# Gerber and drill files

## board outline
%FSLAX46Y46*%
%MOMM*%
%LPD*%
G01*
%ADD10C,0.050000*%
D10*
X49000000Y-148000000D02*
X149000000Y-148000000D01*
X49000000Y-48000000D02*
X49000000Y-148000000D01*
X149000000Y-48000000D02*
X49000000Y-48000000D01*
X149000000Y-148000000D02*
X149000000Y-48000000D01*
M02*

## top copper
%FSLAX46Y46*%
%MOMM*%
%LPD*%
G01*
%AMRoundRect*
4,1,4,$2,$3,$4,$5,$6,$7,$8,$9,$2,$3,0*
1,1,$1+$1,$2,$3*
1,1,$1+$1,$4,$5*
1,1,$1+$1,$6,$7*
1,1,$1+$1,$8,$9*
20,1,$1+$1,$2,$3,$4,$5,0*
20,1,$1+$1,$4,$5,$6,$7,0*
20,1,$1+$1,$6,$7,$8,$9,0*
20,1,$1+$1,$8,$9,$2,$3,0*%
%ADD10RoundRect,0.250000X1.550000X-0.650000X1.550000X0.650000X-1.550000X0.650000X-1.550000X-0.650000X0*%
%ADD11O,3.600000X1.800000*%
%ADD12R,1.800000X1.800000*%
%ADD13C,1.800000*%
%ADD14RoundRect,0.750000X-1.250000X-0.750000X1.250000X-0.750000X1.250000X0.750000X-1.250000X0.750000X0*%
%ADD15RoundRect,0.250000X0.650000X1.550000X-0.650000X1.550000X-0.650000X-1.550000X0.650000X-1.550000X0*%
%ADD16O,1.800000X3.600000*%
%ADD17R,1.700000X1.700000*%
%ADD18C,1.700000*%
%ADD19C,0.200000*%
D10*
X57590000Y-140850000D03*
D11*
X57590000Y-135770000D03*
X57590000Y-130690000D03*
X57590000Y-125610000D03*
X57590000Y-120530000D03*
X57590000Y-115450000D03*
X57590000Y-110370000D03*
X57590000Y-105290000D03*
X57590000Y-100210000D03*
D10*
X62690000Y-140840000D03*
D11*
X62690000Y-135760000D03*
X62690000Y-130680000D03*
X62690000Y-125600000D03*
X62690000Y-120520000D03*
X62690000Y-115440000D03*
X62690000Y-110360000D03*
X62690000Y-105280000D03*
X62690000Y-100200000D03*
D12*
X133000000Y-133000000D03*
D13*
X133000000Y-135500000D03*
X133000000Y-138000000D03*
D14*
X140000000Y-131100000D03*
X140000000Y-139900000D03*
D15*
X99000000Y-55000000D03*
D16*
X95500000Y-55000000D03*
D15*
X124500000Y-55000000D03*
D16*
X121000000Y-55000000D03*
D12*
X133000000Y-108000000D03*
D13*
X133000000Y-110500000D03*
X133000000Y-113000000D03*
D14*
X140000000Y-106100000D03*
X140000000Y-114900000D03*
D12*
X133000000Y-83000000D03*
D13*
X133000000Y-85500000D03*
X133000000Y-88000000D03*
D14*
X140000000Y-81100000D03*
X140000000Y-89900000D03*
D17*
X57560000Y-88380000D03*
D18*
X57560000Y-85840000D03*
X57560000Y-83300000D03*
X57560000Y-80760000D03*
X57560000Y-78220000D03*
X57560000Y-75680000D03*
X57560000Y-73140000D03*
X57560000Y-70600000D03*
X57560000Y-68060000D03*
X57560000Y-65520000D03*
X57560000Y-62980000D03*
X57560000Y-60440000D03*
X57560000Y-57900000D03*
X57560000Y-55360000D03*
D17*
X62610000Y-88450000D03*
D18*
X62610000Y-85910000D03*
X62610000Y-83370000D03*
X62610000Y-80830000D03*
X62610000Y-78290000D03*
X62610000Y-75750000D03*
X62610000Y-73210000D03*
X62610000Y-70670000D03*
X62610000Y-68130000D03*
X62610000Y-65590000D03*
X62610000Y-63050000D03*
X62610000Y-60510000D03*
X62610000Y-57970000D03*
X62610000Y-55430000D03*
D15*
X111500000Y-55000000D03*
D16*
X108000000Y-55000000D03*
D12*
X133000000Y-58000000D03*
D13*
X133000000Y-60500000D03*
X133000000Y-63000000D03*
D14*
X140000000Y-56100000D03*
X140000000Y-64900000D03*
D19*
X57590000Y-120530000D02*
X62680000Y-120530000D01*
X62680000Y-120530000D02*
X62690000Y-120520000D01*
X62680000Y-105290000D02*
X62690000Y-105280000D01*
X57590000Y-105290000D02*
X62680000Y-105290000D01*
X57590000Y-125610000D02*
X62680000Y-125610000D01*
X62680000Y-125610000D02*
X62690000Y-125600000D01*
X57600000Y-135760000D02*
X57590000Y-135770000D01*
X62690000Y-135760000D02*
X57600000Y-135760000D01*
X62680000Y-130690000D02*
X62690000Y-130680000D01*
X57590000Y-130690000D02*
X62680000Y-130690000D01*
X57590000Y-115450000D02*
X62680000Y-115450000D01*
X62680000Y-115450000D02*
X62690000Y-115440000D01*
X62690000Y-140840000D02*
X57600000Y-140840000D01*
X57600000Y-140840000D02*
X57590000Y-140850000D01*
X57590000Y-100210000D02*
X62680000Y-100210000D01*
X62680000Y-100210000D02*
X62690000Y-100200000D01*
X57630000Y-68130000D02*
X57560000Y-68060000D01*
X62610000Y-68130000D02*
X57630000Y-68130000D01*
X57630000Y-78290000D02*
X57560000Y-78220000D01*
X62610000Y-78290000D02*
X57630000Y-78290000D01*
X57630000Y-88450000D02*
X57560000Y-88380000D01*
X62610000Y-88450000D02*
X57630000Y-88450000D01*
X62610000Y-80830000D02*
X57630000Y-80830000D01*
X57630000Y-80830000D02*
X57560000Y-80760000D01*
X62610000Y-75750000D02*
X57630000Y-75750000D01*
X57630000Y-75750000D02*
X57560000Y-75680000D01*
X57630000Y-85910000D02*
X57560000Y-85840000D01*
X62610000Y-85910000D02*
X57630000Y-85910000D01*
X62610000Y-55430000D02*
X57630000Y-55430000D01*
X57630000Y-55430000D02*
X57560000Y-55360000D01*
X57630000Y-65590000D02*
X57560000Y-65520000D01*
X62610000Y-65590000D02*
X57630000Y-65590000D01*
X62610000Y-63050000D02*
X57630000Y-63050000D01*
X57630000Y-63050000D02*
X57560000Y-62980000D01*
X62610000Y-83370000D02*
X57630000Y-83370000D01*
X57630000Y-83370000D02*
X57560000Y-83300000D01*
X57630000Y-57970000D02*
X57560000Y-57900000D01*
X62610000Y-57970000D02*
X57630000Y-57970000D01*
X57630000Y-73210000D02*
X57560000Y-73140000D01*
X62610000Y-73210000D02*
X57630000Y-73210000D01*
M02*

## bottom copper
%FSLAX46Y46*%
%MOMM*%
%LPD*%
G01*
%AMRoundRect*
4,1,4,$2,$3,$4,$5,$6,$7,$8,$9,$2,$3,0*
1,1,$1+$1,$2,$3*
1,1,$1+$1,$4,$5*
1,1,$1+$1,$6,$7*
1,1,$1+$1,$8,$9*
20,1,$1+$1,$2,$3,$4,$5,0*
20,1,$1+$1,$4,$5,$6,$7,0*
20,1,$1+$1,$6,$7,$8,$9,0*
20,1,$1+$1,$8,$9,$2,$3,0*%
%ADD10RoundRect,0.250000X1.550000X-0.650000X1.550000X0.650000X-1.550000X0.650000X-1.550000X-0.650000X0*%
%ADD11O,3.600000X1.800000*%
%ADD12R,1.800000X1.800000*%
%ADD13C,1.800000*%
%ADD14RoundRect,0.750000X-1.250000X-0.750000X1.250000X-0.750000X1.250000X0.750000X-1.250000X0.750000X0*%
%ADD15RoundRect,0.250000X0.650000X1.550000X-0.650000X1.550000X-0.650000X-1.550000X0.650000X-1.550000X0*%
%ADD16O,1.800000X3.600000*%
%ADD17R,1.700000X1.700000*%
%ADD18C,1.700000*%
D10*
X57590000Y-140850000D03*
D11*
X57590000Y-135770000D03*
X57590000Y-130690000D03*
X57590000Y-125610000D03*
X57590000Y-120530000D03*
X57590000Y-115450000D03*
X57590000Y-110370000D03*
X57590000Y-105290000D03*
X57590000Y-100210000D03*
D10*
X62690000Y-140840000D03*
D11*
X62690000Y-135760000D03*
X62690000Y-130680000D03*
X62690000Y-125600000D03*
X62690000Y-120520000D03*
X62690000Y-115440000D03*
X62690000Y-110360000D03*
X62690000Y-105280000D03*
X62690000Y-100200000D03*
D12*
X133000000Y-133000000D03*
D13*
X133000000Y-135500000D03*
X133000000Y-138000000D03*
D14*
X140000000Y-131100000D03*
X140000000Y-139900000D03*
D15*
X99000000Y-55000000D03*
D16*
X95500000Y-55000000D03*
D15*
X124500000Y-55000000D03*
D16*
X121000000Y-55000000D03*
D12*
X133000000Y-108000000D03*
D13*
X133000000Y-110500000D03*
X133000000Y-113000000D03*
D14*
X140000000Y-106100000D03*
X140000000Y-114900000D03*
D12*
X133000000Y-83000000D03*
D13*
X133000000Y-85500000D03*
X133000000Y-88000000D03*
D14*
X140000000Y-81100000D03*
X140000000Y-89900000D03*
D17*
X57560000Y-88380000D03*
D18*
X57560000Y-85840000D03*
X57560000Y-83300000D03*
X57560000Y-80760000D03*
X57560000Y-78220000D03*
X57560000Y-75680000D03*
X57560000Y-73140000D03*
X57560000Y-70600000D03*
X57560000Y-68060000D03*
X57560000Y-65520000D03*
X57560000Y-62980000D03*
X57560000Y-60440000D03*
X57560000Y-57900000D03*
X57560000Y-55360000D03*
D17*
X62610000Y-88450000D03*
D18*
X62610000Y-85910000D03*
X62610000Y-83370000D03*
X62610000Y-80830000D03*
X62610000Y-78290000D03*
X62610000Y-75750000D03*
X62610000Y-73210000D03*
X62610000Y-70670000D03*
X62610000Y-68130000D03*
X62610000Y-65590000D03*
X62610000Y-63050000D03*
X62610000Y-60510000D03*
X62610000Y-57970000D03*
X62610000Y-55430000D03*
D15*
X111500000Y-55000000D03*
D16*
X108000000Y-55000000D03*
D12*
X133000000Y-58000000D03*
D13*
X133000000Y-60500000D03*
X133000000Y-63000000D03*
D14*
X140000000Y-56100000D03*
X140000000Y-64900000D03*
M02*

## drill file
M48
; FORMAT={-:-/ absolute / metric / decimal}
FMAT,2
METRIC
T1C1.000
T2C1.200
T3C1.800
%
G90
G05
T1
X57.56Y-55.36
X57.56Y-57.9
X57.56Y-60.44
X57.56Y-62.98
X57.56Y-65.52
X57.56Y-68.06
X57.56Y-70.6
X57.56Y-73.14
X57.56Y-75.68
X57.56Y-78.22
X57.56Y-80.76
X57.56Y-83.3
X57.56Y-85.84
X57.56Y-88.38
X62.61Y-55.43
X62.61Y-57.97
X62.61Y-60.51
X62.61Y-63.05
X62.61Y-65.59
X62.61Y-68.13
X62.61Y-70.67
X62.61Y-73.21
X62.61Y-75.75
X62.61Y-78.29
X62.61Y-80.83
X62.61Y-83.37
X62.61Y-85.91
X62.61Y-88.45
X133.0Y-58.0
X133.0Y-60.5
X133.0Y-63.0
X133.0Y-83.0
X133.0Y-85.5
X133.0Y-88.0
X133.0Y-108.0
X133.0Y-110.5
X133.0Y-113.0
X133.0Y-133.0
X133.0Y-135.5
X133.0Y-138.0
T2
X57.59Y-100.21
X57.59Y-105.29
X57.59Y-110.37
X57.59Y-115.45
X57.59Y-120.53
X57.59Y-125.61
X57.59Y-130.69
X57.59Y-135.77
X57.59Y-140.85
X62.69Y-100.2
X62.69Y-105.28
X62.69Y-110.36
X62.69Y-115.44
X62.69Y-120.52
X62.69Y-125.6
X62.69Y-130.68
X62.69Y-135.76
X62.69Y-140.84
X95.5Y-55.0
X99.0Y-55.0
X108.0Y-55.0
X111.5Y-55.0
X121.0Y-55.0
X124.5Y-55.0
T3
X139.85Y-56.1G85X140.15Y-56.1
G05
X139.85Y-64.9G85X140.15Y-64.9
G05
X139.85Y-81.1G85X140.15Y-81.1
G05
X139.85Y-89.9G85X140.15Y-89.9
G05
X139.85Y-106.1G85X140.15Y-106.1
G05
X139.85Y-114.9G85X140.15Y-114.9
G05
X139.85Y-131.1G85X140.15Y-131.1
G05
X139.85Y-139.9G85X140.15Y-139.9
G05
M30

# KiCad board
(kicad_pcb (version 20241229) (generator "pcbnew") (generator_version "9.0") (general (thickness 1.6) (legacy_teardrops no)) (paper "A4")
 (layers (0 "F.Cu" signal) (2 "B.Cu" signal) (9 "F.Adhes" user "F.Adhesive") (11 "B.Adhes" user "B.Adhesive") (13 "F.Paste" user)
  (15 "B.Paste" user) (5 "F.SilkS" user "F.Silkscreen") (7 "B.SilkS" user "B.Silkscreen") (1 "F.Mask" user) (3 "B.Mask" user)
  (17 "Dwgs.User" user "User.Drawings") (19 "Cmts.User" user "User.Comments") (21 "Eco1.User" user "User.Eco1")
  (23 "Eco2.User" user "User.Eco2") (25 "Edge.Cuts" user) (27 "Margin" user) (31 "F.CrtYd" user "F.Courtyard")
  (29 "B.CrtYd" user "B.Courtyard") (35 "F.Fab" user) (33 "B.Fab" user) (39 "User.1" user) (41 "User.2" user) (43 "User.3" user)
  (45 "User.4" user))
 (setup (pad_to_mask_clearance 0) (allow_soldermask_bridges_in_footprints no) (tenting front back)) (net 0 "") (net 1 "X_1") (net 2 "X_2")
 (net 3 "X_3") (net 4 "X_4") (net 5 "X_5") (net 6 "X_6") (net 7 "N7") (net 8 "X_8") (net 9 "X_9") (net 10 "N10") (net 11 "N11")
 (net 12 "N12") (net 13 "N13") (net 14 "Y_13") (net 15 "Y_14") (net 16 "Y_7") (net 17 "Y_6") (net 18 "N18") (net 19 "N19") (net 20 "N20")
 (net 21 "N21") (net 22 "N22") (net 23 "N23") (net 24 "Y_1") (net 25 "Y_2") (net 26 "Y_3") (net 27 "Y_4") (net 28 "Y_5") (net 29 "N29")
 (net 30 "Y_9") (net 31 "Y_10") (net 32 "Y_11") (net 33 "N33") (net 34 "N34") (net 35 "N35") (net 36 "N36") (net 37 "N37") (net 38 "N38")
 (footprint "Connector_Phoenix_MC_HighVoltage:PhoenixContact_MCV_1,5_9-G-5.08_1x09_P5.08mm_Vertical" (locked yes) (layer "F.Cu")
  (at 57.59 140.85 90)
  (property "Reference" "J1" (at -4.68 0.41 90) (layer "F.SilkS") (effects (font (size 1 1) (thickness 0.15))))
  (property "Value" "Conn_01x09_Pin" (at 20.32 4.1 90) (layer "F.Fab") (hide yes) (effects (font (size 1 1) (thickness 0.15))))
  (pad "1" thru_hole roundrect (at 0 0 90) (size 1.8 3.6) (drill 1.2) (layers "*.Cu" "*.Mask") (remove_unused_layers no)
   (roundrect_rratio 0.138889) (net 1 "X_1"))
  (pad "2" thru_hole oval (at 5.08 0 90) (size 1.8 3.6) (drill 1.2) (layers "*.Cu" "*.Mask") (remove_unused_layers no) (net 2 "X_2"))
  (pad "3" thru_hole oval (at 10.16 0 90) (size 1.8 3.6) (drill 1.2) (layers "*.Cu" "*.Mask") (remove_unused_layers no) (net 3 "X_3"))
  (pad "4" thru_hole oval (at 15.24 0 90) (size 1.8 3.6) (drill 1.2) (layers "*.Cu" "*.Mask") (remove_unused_layers no) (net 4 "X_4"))
  (pad "5" thru_hole oval (at 20.32 0 90) (size 1.8 3.6) (drill 1.2) (layers "*.Cu" "*.Mask") (remove_unused_layers no) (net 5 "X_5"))
  (pad "6" thru_hole oval (at 25.4 0 90) (size 1.8 3.6) (drill 1.2) (layers "*.Cu" "*.Mask") (remove_unused_layers no) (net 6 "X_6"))
  (pad "7" thru_hole oval (at 30.48 0 90) (size 1.8 3.6) (drill 1.2) (layers "*.Cu" "*.Mask") (remove_unused_layers no) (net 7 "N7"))
  (pad "8" thru_hole oval (at 35.56 0 90) (size 1.8 3.6) (drill 1.2) (layers "*.Cu" "*.Mask") (remove_unused_layers no) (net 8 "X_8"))
  (pad "9" thru_hole oval (at 40.64 0 90) (size 1.8 3.6) (drill 1.2) (layers "*.Cu" "*.Mask") (remove_unused_layers no) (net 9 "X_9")))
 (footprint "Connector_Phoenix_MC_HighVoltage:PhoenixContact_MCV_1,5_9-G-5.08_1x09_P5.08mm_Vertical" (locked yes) (layer "F.Cu")
  (at 62.69 140.84 90)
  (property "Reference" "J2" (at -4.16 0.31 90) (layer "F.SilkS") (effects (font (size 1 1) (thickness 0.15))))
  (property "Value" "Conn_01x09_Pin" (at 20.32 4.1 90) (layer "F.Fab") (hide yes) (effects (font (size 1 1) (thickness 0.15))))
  (pad "1" thru_hole roundrect (at 0 0 90) (size 1.8 3.6) (drill 1.2) (layers "*.Cu" "*.Mask") (remove_unused_layers no)
   (roundrect_rratio 0.138889) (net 1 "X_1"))
  (pad "2" thru_hole oval (at 5.08 0 90) (size 1.8 3.6) (drill 1.2) (layers "*.Cu" "*.Mask") (remove_unused_layers no) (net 2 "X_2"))
  (pad "3" thru_hole oval (at 10.16 0 90) (size 1.8 3.6) (drill 1.2) (layers "*.Cu" "*.Mask") (remove_unused_layers no) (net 3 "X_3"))
  (pad "4" thru_hole oval (at 15.24 0 90) (size 1.8 3.6) (drill 1.2) (layers "*.Cu" "*.Mask") (remove_unused_layers no) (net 4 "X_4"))
  (pad "5" thru_hole oval (at 20.32 0 90) (size 1.8 3.6) (drill 1.2) (layers "*.Cu" "*.Mask") (remove_unused_layers no) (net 5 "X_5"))
  (pad "6" thru_hole oval (at 25.4 0 90) (size 1.8 3.6) (drill 1.2) (layers "*.Cu" "*.Mask") (remove_unused_layers no) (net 6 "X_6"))
  (pad "7" thru_hole oval (at 30.48 0 90) (size 1.8 3.6) (drill 1.2) (layers "*.Cu" "*.Mask") (remove_unused_layers no) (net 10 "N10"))
  (pad "8" thru_hole oval (at 35.56 0 90) (size 1.8 3.6) (drill 1.2) (layers "*.Cu" "*.Mask") (remove_unused_layers no) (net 8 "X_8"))
  (pad "9" thru_hole oval (at 40.64 0 90) (size 1.8 3.6) (drill 1.2) (layers "*.Cu" "*.Mask") (remove_unused_layers no) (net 9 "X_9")))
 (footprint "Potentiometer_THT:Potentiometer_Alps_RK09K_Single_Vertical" (layer "F.Cu") (at 133 133)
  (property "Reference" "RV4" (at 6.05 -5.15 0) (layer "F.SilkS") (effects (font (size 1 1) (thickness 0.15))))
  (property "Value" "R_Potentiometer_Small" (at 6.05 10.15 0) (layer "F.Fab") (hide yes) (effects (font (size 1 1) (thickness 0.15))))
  (pad "1" thru_hole rect (at 0 0) (size 1.8 1.8) (drill 1) (layers "*.Cu" "*.Mask") (remove_unused_layers no) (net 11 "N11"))
  (pad "2" thru_hole circle (at 0 2.5) (size 1.8 1.8) (drill 1) (layers "*.Cu" "*.Mask") (remove_unused_layers no) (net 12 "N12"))
  (pad "3" thru_hole circle (at 0 5) (size 1.8 1.8) (drill 1) (layers "*.Cu" "*.Mask") (remove_unused_layers no) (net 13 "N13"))
  (pad "MP" thru_hole roundrect (at 7 -1.9) (size 4 3) (drill oval 2.1 1.8) (layers "*.Cu" "*.Mask") (remove_unused_layers no)
   (roundrect_rratio 0.25))
  (pad "MP" thru_hole roundrect (at 7 6.9) (size 4 3) (drill oval 2.1 1.8) (layers "*.Cu" "*.Mask") (remove_unused_layers no)
   (roundrect_rratio 0.25)))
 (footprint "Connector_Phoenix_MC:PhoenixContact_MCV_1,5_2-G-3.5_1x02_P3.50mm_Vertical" (layer "F.Cu") (at 99 55 180)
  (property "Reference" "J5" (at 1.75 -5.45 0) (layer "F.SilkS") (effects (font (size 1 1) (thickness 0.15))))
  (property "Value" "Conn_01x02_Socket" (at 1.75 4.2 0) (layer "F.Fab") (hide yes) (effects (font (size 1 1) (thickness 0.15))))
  (pad "1" thru_hole roundrect (at 0 0 180) (size 1.8 3.6) (drill 1.2) (layers "*.Cu" "*.Mask") (remove_unused_layers no)
   (roundrect_rratio 0.138889) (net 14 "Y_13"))
  (pad "2" thru_hole oval (at 3.5 0 180) (size 1.8 3.6) (drill 1.2) (layers "*.Cu" "*.Mask") (remove_unused_layers no) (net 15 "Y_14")))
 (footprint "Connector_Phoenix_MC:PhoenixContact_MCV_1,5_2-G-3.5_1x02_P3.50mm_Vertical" (layer "F.Cu") (at 124.5 55 180)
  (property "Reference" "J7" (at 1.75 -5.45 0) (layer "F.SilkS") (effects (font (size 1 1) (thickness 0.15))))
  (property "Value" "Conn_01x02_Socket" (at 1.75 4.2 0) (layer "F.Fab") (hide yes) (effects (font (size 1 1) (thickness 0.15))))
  (pad "1" thru_hole roundrect (at 0 0 180) (size 1.8 3.6) (drill 1.2) (layers "*.Cu" "*.Mask") (remove_unused_layers no)
   (roundrect_rratio 0.138889) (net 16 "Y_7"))
  (pad "2" thru_hole oval (at 3.5 0 180) (size 1.8 3.6) (drill 1.2) (layers "*.Cu" "*.Mask") (remove_unused_layers no) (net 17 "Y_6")))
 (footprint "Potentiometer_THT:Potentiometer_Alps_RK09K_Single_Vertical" (layer "F.Cu") (at 133 108)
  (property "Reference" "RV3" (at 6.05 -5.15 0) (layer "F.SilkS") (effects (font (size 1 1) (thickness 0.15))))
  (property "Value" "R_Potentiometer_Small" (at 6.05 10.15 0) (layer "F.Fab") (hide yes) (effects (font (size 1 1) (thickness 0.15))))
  (pad "1" thru_hole rect (at 0 0) (size 1.8 1.8) (drill 1) (layers "*.Cu" "*.Mask") (remove_unused_layers no) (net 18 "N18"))
  (pad "2" thru_hole circle (at 0 2.5) (size 1.8 1.8) (drill 1) (layers "*.Cu" "*.Mask") (remove_unused_layers no) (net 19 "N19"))
  (pad "3" thru_hole circle (at 0 5) (size 1.8 1.8) (drill 1) (layers "*.Cu" "*.Mask") (remove_unused_layers no) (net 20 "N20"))
  (pad "MP" thru_hole roundrect (at 7 -1.9) (size 4 3) (drill oval 2.1 1.8) (layers "*.Cu" "*.Mask") (remove_unused_layers no)
   (roundrect_rratio 0.25))
  (pad "MP" thru_hole roundrect (at 7 6.9) (size 4 3) (drill oval 2.1 1.8) (layers "*.Cu" "*.Mask") (remove_unused_layers no)
   (roundrect_rratio 0.25)))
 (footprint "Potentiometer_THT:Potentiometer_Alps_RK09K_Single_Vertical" (layer "F.Cu") (at 133 83)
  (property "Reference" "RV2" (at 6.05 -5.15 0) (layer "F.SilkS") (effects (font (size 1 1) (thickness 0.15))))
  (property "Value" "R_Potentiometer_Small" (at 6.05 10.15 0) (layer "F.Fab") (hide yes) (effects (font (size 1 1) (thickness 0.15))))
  (pad "1" thru_hole rect (at 0 0) (size 1.8 1.8) (drill 1) (layers "*.Cu" "*.Mask") (remove_unused_layers no) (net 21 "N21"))
  (pad "2" thru_hole circle (at 0 2.5) (size 1.8 1.8) (drill 1) (layers "*.Cu" "*.Mask") (remove_unused_layers no) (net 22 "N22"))
  (pad "3" thru_hole circle (at 0 5) (size 1.8 1.8) (drill 1) (layers "*.Cu" "*.Mask") (remove_unused_layers no) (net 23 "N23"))
  (pad "MP" thru_hole roundrect (at 7 -1.9) (size 4 3) (drill oval 2.1 1.8) (layers "*.Cu" "*.Mask") (remove_unused_layers no)
   (roundrect_rratio 0.25))
  (pad "MP" thru_hole roundrect (at 7 6.9) (size 4 3) (drill oval 2.1 1.8) (layers "*.Cu" "*.Mask") (remove_unused_layers no)
   (roundrect_rratio 0.25)))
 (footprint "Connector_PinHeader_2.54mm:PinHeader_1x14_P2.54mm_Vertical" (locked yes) (layer "F.Cu") (at 57.56 88.38 180)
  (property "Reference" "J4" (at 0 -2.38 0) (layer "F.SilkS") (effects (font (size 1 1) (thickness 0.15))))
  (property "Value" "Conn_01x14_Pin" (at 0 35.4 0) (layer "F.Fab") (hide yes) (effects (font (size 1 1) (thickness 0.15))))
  (pad "1" thru_hole rect (at 0 0 180) (size 1.7 1.7) (drill 1) (layers "*.Cu" "*.Mask") (remove_unused_layers no) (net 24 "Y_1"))
  (pad "2" thru_hole circle (at 0 2.54 180) (size 1.7 1.7) (drill 1) (layers "*.Cu" "*.Mask") (remove_unused_layers no) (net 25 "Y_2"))
  (pad "3" thru_hole circle (at 0 5.08 180) (size 1.7 1.7) (drill 1) (layers "*.Cu" "*.Mask") (remove_unused_layers no) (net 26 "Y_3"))
  (pad "4" thru_hole circle (at 0 7.62 180) (size 1.7 1.7) (drill 1) (layers "*.Cu" "*.Mask") (remove_unused_layers no) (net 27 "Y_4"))
  (pad "5" thru_hole circle (at 0 10.16 180) (size 1.7 1.7) (drill 1) (layers "*.Cu" "*.Mask") (remove_unused_layers no) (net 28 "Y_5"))
  (pad "6" thru_hole circle (at 0 12.7 180) (size 1.7 1.7) (drill 1) (layers "*.Cu" "*.Mask") (remove_unused_layers no) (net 17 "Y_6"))
  (pad "7" thru_hole circle (at 0 15.24 180) (size 1.7 1.7) (drill 1) (layers "*.Cu" "*.Mask") (remove_unused_layers no) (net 16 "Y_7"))
  (pad "8" thru_hole circle (at 0 17.78 180) (size 1.7 1.7) (drill 1) (layers "*.Cu" "*.Mask") (remove_unused_layers no) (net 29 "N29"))
  (pad "9" thru_hole circle (at 0 20.32 180) (size 1.7 1.7) (drill 1) (layers "*.Cu" "*.Mask") (remove_unused_layers no) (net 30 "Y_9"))
  (pad "10" thru_hole circle (at 0 22.86 180) (size 1.7 1.7) (drill 1) (layers "*.Cu" "*.Mask") (remove_unused_layers no) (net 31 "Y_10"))
  (pad "11" thru_hole circle (at 0 25.4 180) (size 1.7 1.7) (drill 1) (layers "*.Cu" "*.Mask") (remove_unused_layers no) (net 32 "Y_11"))
  (pad "12" thru_hole circle (at 0 27.94 180) (size 1.7 1.7) (drill 1) (layers "*.Cu" "*.Mask") (remove_unused_layers no) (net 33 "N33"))
  (pad "13" thru_hole circle (at 0 30.48 180) (size 1.7 1.7) (drill 1) (layers "*.Cu" "*.Mask") (remove_unused_layers no) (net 14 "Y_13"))
  (pad "14" thru_hole circle (at 0 33.02 180) (size 1.7 1.7) (drill 1) (layers "*.Cu" "*.Mask") (remove_unused_layers no) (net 15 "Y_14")))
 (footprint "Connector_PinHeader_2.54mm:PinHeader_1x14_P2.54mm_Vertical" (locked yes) (layer "F.Cu") (at 62.61 88.45 180)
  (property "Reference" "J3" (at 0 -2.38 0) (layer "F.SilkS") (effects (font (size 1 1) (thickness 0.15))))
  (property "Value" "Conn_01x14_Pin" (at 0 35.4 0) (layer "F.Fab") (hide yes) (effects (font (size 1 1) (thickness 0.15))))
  (pad "1" thru_hole rect (at 0 0 180) (size 1.7 1.7) (drill 1) (layers "*.Cu" "*.Mask") (remove_unused_layers no) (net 24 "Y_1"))
  (pad "2" thru_hole circle (at 0 2.54 180) (size 1.7 1.7) (drill 1) (layers "*.Cu" "*.Mask") (remove_unused_layers no) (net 25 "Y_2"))
  (pad "3" thru_hole circle (at 0 5.08 180) (size 1.7 1.7) (drill 1) (layers "*.Cu" "*.Mask") (remove_unused_layers no) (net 26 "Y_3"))
  (pad "4" thru_hole circle (at 0 7.62 180) (size 1.7 1.7) (drill 1) (layers "*.Cu" "*.Mask") (remove_unused_layers no) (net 27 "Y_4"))
  (pad "5" thru_hole circle (at 0 10.16 180) (size 1.7 1.7) (drill 1) (layers "*.Cu" "*.Mask") (remove_unused_layers no) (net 28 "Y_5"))
  (pad "6" thru_hole circle (at 0 12.7 180) (size 1.7 1.7) (drill 1) (layers "*.Cu" "*.Mask") (remove_unused_layers no) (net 17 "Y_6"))
  (pad "7" thru_hole circle (at 0 15.24 180) (size 1.7 1.7) (drill 1) (layers "*.Cu" "*.Mask") (remove_unused_layers no) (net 16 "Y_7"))
  (pad "8" thru_hole circle (at 0 17.78 180) (size 1.7 1.7) (drill 1) (layers "*.Cu" "*.Mask") (remove_unused_layers no) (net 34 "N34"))
  (pad "9" thru_hole circle (at 0 20.32 180) (size 1.7 1.7) (drill 1) (layers "*.Cu" "*.Mask") (remove_unused_layers no) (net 30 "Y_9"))
  (pad "10" thru_hole circle (at 0 22.86 180) (size 1.7 1.7) (drill 1) (layers "*.Cu" "*.Mask") (remove_unused_layers no) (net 31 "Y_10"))
  (pad "11" thru_hole circle (at 0 25.4 180) (size 1.7 1.7) (drill 1) (layers "*.Cu" "*.Mask") (remove_unused_layers no) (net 32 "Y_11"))
  (pad "12" thru_hole circle (at 0 27.94 180) (size 1.7 1.7) (drill 1) (layers "*.Cu" "*.Mask") (remove_unused_layers no) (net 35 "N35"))
  (pad "13" thru_hole circle (at 0 30.48 180) (size 1.7 1.7) (drill 1) (layers "*.Cu" "*.Mask") (remove_unused_layers no) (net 14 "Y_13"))
  (pad "14" thru_hole circle (at 0 33.02 180) (size 1.7 1.7) (drill 1) (layers "*.Cu" "*.Mask") (remove_unused_layers no) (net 15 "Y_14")))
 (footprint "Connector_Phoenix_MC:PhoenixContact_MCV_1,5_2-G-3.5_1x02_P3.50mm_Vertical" (layer "F.Cu") (at 111.5 55 180)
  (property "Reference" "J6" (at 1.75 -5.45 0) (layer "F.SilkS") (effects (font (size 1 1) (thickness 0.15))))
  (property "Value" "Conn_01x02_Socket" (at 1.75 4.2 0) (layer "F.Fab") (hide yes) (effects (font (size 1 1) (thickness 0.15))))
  (pad "1" thru_hole roundrect (at 0 0 180) (size 1.8 3.6) (drill 1.2) (layers "*.Cu" "*.Mask") (remove_unused_layers no)
   (roundrect_rratio 0.138889) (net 31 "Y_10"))
  (pad "2" thru_hole oval (at 3.5 0 180) (size 1.8 3.6) (drill 1.2) (layers "*.Cu" "*.Mask") (remove_unused_layers no) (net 30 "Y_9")))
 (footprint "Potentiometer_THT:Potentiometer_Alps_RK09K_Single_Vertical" (layer "F.Cu") (at 133 58)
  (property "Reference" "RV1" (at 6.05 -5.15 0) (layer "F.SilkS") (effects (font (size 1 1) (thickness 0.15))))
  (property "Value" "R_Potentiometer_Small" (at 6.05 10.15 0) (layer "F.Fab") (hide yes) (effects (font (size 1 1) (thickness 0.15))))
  (pad "1" thru_hole rect (at 0 0) (size 1.8 1.8) (drill 1) (layers "*.Cu" "*.Mask") (remove_unused_layers no) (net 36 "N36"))
  (pad "2" thru_hole circle (at 0 2.5) (size 1.8 1.8) (drill 1) (layers "*.Cu" "*.Mask") (remove_unused_layers no) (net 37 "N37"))
  (pad "3" thru_hole circle (at 0 5) (size 1.8 1.8) (drill 1) (layers "*.Cu" "*.Mask") (remove_unused_layers no) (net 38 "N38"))
  (pad "MP" thru_hole roundrect (at 7 -1.9) (size 4 3) (drill oval 2.1 1.8) (layers "*.Cu" "*.Mask") (remove_unused_layers no)
   (roundrect_rratio 0.25))
  (pad "MP" thru_hole roundrect (at 7 6.9) (size 4 3) (drill oval 2.1 1.8) (layers "*.Cu" "*.Mask") (remove_unused_layers no)
   (roundrect_rratio 0.25)))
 (gr_line (start 49 148) (end 149 148) (stroke (width 0.05) (type default)) (locked yes) (layer "Edge.Cuts"))
 (gr_line (start 49 48) (end 49 148) (stroke (width 0.05) (type default)) (locked yes) (layer "Edge.Cuts"))
 (gr_line (start 149 48) (end 49 48) (stroke (width 0.05) (type default)) (locked yes) (layer "Edge.Cuts"))
 (gr_line (start 149 148) (end 149 48) (stroke (width 0.05) (type default)) (locked yes) (layer "Edge.Cuts"))
 (segment (start 57.59 120.53) (end 62.68 120.53) (width 0.2) (locked yes) (layer "F.Cu") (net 5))
 (segment (start 62.68 120.53) (end 62.69 120.52) (width 0.2) (locked yes) (layer "F.Cu") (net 5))
 (segment (start 62.68 105.29) (end 62.69 105.28) (width 0.2) (locked yes) (layer "F.Cu") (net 8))
 (segment (start 57.59 105.29) (end 62.68 105.29) (width 0.2) (locked yes) (layer "F.Cu") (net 8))
 (segment (start 57.59 125.61) (end 62.68 125.61) (width 0.2) (locked yes) (layer "F.Cu") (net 4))
 (segment (start 62.68 125.61) (end 62.69 125.6) (width 0.2) (locked yes) (layer "F.Cu") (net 4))
 (segment (start 57.6 135.76) (end 57.59 135.77) (width 0.2) (locked yes) (layer "F.Cu") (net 2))
 (segment (start 62.69 135.76) (end 57.6 135.76) (width 0.2) (locked yes) (layer "F.Cu") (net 2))
 (segment (start 62.68 130.69) (end 62.69 130.68) (width 0.2) (locked yes) (layer "F.Cu") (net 3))
 (segment (start 57.59 130.69) (end 62.68 130.69) (width 0.2) (locked yes) (layer "F.Cu") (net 3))
 (segment (start 57.59 115.45) (end 62.68 115.45) (width 0.2) (locked yes) (layer "F.Cu") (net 6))
 (segment (start 62.68 115.45) (end 62.69 115.44) (width 0.2) (locked yes) (layer "F.Cu") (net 6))
 (segment (start 62.69 140.84) (end 57.6 140.84) (width 0.2) (locked yes) (layer "F.Cu") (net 1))
 (segment (start 57.6 140.84) (end 57.59 140.85) (width 0.2) (locked yes) (layer "F.Cu") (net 1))
 (segment (start 57.59 100.21) (end 62.68 100.21) (width 0.2) (locked yes) (layer "F.Cu") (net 9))
 (segment (start 62.68 100.21) (end 62.69 100.2) (width 0.2) (locked yes) (layer "F.Cu") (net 9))
 (segment (start 57.63 68.13) (end 57.56 68.06) (width 0.2) (locked yes) (layer "F.Cu") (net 30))
 (segment (start 62.61 68.13) (end 57.63 68.13) (width 0.2) (locked yes) (layer "F.Cu") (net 30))
 (segment (start 57.63 78.29) (end 57.56 78.22) (width 0.2) (locked yes) (layer "F.Cu") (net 28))
 (segment (start 62.61 78.29) (end 57.63 78.29) (width 0.2) (locked yes) (layer "F.Cu") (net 28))
 (segment (start 57.63 88.45) (end 57.56 88.38) (width 0.2) (locked yes) (layer "F.Cu") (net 24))
 (segment (start 62.61 88.45) (end 57.63 88.45) (width 0.2) (locked yes) (layer "F.Cu") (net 24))
 (segment (start 62.61 80.83) (end 57.63 80.83) (width 0.2) (locked yes) (layer "F.Cu") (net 27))
 (segment (start 57.63 80.83) (end 57.56 80.76) (width 0.2) (locked yes) (layer "F.Cu") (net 27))
 (segment (start 62.61 75.75) (end 57.63 75.75) (width 0.2) (locked yes) (layer "F.Cu") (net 17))
 (segment (start 57.63 75.75) (end 57.56 75.68) (width 0.2) (locked yes) (layer "F.Cu") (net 17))
 (segment (start 57.63 85.91) (end 57.56 85.84) (width 0.2) (locked yes) (layer "F.Cu") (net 25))
 (segment (start 62.61 85.91) (end 57.63 85.91) (width 0.2) (locked yes) (layer "F.Cu") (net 25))
 (segment (start 62.61 55.43) (end 57.63 55.43) (width 0.2) (locked yes) (layer "F.Cu") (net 15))
 (segment (start 57.63 55.43) (end 57.56 55.36) (width 0.2) (locked yes) (layer "F.Cu") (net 15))
 (segment (start 57.63 65.59) (end 57.56 65.52) (width 0.2) (locked yes) (layer "F.Cu") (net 31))
 (segment (start 62.61 65.59) (end 57.63 65.59) (width 0.2) (locked yes) (layer "F.Cu") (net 31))
 (segment (start 62.61 63.05) (end 57.63 63.05) (width 0.2) (locked yes) (layer "F.Cu") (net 32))
 (segment (start 57.63 63.05) (end 57.56 62.98) (width 0.2) (locked yes) (layer "F.Cu") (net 32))
 (segment (start 62.61 83.37) (end 57.63 83.37) (width 0.2) (locked yes) (layer "F.Cu") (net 26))
 (segment (start 57.63 83.37) (end 57.56 83.3) (width 0.2) (locked yes) (layer "F.Cu") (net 26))
 (segment (start 57.63 57.97) (end 57.56 57.9) (width 0.2) (locked yes) (layer "F.Cu") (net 14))
 (segment (start 62.61 57.97) (end 57.63 57.97) (width 0.2) (locked yes) (layer "F.Cu") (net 14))
 (segment (start 57.63 73.21) (end 57.56 73.14) (width 0.2) (locked yes) (layer "F.Cu") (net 16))
 (segment (start 62.61 73.21) (end 57.63 73.21) (width 0.2) (locked yes) (layer "F.Cu") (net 16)))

